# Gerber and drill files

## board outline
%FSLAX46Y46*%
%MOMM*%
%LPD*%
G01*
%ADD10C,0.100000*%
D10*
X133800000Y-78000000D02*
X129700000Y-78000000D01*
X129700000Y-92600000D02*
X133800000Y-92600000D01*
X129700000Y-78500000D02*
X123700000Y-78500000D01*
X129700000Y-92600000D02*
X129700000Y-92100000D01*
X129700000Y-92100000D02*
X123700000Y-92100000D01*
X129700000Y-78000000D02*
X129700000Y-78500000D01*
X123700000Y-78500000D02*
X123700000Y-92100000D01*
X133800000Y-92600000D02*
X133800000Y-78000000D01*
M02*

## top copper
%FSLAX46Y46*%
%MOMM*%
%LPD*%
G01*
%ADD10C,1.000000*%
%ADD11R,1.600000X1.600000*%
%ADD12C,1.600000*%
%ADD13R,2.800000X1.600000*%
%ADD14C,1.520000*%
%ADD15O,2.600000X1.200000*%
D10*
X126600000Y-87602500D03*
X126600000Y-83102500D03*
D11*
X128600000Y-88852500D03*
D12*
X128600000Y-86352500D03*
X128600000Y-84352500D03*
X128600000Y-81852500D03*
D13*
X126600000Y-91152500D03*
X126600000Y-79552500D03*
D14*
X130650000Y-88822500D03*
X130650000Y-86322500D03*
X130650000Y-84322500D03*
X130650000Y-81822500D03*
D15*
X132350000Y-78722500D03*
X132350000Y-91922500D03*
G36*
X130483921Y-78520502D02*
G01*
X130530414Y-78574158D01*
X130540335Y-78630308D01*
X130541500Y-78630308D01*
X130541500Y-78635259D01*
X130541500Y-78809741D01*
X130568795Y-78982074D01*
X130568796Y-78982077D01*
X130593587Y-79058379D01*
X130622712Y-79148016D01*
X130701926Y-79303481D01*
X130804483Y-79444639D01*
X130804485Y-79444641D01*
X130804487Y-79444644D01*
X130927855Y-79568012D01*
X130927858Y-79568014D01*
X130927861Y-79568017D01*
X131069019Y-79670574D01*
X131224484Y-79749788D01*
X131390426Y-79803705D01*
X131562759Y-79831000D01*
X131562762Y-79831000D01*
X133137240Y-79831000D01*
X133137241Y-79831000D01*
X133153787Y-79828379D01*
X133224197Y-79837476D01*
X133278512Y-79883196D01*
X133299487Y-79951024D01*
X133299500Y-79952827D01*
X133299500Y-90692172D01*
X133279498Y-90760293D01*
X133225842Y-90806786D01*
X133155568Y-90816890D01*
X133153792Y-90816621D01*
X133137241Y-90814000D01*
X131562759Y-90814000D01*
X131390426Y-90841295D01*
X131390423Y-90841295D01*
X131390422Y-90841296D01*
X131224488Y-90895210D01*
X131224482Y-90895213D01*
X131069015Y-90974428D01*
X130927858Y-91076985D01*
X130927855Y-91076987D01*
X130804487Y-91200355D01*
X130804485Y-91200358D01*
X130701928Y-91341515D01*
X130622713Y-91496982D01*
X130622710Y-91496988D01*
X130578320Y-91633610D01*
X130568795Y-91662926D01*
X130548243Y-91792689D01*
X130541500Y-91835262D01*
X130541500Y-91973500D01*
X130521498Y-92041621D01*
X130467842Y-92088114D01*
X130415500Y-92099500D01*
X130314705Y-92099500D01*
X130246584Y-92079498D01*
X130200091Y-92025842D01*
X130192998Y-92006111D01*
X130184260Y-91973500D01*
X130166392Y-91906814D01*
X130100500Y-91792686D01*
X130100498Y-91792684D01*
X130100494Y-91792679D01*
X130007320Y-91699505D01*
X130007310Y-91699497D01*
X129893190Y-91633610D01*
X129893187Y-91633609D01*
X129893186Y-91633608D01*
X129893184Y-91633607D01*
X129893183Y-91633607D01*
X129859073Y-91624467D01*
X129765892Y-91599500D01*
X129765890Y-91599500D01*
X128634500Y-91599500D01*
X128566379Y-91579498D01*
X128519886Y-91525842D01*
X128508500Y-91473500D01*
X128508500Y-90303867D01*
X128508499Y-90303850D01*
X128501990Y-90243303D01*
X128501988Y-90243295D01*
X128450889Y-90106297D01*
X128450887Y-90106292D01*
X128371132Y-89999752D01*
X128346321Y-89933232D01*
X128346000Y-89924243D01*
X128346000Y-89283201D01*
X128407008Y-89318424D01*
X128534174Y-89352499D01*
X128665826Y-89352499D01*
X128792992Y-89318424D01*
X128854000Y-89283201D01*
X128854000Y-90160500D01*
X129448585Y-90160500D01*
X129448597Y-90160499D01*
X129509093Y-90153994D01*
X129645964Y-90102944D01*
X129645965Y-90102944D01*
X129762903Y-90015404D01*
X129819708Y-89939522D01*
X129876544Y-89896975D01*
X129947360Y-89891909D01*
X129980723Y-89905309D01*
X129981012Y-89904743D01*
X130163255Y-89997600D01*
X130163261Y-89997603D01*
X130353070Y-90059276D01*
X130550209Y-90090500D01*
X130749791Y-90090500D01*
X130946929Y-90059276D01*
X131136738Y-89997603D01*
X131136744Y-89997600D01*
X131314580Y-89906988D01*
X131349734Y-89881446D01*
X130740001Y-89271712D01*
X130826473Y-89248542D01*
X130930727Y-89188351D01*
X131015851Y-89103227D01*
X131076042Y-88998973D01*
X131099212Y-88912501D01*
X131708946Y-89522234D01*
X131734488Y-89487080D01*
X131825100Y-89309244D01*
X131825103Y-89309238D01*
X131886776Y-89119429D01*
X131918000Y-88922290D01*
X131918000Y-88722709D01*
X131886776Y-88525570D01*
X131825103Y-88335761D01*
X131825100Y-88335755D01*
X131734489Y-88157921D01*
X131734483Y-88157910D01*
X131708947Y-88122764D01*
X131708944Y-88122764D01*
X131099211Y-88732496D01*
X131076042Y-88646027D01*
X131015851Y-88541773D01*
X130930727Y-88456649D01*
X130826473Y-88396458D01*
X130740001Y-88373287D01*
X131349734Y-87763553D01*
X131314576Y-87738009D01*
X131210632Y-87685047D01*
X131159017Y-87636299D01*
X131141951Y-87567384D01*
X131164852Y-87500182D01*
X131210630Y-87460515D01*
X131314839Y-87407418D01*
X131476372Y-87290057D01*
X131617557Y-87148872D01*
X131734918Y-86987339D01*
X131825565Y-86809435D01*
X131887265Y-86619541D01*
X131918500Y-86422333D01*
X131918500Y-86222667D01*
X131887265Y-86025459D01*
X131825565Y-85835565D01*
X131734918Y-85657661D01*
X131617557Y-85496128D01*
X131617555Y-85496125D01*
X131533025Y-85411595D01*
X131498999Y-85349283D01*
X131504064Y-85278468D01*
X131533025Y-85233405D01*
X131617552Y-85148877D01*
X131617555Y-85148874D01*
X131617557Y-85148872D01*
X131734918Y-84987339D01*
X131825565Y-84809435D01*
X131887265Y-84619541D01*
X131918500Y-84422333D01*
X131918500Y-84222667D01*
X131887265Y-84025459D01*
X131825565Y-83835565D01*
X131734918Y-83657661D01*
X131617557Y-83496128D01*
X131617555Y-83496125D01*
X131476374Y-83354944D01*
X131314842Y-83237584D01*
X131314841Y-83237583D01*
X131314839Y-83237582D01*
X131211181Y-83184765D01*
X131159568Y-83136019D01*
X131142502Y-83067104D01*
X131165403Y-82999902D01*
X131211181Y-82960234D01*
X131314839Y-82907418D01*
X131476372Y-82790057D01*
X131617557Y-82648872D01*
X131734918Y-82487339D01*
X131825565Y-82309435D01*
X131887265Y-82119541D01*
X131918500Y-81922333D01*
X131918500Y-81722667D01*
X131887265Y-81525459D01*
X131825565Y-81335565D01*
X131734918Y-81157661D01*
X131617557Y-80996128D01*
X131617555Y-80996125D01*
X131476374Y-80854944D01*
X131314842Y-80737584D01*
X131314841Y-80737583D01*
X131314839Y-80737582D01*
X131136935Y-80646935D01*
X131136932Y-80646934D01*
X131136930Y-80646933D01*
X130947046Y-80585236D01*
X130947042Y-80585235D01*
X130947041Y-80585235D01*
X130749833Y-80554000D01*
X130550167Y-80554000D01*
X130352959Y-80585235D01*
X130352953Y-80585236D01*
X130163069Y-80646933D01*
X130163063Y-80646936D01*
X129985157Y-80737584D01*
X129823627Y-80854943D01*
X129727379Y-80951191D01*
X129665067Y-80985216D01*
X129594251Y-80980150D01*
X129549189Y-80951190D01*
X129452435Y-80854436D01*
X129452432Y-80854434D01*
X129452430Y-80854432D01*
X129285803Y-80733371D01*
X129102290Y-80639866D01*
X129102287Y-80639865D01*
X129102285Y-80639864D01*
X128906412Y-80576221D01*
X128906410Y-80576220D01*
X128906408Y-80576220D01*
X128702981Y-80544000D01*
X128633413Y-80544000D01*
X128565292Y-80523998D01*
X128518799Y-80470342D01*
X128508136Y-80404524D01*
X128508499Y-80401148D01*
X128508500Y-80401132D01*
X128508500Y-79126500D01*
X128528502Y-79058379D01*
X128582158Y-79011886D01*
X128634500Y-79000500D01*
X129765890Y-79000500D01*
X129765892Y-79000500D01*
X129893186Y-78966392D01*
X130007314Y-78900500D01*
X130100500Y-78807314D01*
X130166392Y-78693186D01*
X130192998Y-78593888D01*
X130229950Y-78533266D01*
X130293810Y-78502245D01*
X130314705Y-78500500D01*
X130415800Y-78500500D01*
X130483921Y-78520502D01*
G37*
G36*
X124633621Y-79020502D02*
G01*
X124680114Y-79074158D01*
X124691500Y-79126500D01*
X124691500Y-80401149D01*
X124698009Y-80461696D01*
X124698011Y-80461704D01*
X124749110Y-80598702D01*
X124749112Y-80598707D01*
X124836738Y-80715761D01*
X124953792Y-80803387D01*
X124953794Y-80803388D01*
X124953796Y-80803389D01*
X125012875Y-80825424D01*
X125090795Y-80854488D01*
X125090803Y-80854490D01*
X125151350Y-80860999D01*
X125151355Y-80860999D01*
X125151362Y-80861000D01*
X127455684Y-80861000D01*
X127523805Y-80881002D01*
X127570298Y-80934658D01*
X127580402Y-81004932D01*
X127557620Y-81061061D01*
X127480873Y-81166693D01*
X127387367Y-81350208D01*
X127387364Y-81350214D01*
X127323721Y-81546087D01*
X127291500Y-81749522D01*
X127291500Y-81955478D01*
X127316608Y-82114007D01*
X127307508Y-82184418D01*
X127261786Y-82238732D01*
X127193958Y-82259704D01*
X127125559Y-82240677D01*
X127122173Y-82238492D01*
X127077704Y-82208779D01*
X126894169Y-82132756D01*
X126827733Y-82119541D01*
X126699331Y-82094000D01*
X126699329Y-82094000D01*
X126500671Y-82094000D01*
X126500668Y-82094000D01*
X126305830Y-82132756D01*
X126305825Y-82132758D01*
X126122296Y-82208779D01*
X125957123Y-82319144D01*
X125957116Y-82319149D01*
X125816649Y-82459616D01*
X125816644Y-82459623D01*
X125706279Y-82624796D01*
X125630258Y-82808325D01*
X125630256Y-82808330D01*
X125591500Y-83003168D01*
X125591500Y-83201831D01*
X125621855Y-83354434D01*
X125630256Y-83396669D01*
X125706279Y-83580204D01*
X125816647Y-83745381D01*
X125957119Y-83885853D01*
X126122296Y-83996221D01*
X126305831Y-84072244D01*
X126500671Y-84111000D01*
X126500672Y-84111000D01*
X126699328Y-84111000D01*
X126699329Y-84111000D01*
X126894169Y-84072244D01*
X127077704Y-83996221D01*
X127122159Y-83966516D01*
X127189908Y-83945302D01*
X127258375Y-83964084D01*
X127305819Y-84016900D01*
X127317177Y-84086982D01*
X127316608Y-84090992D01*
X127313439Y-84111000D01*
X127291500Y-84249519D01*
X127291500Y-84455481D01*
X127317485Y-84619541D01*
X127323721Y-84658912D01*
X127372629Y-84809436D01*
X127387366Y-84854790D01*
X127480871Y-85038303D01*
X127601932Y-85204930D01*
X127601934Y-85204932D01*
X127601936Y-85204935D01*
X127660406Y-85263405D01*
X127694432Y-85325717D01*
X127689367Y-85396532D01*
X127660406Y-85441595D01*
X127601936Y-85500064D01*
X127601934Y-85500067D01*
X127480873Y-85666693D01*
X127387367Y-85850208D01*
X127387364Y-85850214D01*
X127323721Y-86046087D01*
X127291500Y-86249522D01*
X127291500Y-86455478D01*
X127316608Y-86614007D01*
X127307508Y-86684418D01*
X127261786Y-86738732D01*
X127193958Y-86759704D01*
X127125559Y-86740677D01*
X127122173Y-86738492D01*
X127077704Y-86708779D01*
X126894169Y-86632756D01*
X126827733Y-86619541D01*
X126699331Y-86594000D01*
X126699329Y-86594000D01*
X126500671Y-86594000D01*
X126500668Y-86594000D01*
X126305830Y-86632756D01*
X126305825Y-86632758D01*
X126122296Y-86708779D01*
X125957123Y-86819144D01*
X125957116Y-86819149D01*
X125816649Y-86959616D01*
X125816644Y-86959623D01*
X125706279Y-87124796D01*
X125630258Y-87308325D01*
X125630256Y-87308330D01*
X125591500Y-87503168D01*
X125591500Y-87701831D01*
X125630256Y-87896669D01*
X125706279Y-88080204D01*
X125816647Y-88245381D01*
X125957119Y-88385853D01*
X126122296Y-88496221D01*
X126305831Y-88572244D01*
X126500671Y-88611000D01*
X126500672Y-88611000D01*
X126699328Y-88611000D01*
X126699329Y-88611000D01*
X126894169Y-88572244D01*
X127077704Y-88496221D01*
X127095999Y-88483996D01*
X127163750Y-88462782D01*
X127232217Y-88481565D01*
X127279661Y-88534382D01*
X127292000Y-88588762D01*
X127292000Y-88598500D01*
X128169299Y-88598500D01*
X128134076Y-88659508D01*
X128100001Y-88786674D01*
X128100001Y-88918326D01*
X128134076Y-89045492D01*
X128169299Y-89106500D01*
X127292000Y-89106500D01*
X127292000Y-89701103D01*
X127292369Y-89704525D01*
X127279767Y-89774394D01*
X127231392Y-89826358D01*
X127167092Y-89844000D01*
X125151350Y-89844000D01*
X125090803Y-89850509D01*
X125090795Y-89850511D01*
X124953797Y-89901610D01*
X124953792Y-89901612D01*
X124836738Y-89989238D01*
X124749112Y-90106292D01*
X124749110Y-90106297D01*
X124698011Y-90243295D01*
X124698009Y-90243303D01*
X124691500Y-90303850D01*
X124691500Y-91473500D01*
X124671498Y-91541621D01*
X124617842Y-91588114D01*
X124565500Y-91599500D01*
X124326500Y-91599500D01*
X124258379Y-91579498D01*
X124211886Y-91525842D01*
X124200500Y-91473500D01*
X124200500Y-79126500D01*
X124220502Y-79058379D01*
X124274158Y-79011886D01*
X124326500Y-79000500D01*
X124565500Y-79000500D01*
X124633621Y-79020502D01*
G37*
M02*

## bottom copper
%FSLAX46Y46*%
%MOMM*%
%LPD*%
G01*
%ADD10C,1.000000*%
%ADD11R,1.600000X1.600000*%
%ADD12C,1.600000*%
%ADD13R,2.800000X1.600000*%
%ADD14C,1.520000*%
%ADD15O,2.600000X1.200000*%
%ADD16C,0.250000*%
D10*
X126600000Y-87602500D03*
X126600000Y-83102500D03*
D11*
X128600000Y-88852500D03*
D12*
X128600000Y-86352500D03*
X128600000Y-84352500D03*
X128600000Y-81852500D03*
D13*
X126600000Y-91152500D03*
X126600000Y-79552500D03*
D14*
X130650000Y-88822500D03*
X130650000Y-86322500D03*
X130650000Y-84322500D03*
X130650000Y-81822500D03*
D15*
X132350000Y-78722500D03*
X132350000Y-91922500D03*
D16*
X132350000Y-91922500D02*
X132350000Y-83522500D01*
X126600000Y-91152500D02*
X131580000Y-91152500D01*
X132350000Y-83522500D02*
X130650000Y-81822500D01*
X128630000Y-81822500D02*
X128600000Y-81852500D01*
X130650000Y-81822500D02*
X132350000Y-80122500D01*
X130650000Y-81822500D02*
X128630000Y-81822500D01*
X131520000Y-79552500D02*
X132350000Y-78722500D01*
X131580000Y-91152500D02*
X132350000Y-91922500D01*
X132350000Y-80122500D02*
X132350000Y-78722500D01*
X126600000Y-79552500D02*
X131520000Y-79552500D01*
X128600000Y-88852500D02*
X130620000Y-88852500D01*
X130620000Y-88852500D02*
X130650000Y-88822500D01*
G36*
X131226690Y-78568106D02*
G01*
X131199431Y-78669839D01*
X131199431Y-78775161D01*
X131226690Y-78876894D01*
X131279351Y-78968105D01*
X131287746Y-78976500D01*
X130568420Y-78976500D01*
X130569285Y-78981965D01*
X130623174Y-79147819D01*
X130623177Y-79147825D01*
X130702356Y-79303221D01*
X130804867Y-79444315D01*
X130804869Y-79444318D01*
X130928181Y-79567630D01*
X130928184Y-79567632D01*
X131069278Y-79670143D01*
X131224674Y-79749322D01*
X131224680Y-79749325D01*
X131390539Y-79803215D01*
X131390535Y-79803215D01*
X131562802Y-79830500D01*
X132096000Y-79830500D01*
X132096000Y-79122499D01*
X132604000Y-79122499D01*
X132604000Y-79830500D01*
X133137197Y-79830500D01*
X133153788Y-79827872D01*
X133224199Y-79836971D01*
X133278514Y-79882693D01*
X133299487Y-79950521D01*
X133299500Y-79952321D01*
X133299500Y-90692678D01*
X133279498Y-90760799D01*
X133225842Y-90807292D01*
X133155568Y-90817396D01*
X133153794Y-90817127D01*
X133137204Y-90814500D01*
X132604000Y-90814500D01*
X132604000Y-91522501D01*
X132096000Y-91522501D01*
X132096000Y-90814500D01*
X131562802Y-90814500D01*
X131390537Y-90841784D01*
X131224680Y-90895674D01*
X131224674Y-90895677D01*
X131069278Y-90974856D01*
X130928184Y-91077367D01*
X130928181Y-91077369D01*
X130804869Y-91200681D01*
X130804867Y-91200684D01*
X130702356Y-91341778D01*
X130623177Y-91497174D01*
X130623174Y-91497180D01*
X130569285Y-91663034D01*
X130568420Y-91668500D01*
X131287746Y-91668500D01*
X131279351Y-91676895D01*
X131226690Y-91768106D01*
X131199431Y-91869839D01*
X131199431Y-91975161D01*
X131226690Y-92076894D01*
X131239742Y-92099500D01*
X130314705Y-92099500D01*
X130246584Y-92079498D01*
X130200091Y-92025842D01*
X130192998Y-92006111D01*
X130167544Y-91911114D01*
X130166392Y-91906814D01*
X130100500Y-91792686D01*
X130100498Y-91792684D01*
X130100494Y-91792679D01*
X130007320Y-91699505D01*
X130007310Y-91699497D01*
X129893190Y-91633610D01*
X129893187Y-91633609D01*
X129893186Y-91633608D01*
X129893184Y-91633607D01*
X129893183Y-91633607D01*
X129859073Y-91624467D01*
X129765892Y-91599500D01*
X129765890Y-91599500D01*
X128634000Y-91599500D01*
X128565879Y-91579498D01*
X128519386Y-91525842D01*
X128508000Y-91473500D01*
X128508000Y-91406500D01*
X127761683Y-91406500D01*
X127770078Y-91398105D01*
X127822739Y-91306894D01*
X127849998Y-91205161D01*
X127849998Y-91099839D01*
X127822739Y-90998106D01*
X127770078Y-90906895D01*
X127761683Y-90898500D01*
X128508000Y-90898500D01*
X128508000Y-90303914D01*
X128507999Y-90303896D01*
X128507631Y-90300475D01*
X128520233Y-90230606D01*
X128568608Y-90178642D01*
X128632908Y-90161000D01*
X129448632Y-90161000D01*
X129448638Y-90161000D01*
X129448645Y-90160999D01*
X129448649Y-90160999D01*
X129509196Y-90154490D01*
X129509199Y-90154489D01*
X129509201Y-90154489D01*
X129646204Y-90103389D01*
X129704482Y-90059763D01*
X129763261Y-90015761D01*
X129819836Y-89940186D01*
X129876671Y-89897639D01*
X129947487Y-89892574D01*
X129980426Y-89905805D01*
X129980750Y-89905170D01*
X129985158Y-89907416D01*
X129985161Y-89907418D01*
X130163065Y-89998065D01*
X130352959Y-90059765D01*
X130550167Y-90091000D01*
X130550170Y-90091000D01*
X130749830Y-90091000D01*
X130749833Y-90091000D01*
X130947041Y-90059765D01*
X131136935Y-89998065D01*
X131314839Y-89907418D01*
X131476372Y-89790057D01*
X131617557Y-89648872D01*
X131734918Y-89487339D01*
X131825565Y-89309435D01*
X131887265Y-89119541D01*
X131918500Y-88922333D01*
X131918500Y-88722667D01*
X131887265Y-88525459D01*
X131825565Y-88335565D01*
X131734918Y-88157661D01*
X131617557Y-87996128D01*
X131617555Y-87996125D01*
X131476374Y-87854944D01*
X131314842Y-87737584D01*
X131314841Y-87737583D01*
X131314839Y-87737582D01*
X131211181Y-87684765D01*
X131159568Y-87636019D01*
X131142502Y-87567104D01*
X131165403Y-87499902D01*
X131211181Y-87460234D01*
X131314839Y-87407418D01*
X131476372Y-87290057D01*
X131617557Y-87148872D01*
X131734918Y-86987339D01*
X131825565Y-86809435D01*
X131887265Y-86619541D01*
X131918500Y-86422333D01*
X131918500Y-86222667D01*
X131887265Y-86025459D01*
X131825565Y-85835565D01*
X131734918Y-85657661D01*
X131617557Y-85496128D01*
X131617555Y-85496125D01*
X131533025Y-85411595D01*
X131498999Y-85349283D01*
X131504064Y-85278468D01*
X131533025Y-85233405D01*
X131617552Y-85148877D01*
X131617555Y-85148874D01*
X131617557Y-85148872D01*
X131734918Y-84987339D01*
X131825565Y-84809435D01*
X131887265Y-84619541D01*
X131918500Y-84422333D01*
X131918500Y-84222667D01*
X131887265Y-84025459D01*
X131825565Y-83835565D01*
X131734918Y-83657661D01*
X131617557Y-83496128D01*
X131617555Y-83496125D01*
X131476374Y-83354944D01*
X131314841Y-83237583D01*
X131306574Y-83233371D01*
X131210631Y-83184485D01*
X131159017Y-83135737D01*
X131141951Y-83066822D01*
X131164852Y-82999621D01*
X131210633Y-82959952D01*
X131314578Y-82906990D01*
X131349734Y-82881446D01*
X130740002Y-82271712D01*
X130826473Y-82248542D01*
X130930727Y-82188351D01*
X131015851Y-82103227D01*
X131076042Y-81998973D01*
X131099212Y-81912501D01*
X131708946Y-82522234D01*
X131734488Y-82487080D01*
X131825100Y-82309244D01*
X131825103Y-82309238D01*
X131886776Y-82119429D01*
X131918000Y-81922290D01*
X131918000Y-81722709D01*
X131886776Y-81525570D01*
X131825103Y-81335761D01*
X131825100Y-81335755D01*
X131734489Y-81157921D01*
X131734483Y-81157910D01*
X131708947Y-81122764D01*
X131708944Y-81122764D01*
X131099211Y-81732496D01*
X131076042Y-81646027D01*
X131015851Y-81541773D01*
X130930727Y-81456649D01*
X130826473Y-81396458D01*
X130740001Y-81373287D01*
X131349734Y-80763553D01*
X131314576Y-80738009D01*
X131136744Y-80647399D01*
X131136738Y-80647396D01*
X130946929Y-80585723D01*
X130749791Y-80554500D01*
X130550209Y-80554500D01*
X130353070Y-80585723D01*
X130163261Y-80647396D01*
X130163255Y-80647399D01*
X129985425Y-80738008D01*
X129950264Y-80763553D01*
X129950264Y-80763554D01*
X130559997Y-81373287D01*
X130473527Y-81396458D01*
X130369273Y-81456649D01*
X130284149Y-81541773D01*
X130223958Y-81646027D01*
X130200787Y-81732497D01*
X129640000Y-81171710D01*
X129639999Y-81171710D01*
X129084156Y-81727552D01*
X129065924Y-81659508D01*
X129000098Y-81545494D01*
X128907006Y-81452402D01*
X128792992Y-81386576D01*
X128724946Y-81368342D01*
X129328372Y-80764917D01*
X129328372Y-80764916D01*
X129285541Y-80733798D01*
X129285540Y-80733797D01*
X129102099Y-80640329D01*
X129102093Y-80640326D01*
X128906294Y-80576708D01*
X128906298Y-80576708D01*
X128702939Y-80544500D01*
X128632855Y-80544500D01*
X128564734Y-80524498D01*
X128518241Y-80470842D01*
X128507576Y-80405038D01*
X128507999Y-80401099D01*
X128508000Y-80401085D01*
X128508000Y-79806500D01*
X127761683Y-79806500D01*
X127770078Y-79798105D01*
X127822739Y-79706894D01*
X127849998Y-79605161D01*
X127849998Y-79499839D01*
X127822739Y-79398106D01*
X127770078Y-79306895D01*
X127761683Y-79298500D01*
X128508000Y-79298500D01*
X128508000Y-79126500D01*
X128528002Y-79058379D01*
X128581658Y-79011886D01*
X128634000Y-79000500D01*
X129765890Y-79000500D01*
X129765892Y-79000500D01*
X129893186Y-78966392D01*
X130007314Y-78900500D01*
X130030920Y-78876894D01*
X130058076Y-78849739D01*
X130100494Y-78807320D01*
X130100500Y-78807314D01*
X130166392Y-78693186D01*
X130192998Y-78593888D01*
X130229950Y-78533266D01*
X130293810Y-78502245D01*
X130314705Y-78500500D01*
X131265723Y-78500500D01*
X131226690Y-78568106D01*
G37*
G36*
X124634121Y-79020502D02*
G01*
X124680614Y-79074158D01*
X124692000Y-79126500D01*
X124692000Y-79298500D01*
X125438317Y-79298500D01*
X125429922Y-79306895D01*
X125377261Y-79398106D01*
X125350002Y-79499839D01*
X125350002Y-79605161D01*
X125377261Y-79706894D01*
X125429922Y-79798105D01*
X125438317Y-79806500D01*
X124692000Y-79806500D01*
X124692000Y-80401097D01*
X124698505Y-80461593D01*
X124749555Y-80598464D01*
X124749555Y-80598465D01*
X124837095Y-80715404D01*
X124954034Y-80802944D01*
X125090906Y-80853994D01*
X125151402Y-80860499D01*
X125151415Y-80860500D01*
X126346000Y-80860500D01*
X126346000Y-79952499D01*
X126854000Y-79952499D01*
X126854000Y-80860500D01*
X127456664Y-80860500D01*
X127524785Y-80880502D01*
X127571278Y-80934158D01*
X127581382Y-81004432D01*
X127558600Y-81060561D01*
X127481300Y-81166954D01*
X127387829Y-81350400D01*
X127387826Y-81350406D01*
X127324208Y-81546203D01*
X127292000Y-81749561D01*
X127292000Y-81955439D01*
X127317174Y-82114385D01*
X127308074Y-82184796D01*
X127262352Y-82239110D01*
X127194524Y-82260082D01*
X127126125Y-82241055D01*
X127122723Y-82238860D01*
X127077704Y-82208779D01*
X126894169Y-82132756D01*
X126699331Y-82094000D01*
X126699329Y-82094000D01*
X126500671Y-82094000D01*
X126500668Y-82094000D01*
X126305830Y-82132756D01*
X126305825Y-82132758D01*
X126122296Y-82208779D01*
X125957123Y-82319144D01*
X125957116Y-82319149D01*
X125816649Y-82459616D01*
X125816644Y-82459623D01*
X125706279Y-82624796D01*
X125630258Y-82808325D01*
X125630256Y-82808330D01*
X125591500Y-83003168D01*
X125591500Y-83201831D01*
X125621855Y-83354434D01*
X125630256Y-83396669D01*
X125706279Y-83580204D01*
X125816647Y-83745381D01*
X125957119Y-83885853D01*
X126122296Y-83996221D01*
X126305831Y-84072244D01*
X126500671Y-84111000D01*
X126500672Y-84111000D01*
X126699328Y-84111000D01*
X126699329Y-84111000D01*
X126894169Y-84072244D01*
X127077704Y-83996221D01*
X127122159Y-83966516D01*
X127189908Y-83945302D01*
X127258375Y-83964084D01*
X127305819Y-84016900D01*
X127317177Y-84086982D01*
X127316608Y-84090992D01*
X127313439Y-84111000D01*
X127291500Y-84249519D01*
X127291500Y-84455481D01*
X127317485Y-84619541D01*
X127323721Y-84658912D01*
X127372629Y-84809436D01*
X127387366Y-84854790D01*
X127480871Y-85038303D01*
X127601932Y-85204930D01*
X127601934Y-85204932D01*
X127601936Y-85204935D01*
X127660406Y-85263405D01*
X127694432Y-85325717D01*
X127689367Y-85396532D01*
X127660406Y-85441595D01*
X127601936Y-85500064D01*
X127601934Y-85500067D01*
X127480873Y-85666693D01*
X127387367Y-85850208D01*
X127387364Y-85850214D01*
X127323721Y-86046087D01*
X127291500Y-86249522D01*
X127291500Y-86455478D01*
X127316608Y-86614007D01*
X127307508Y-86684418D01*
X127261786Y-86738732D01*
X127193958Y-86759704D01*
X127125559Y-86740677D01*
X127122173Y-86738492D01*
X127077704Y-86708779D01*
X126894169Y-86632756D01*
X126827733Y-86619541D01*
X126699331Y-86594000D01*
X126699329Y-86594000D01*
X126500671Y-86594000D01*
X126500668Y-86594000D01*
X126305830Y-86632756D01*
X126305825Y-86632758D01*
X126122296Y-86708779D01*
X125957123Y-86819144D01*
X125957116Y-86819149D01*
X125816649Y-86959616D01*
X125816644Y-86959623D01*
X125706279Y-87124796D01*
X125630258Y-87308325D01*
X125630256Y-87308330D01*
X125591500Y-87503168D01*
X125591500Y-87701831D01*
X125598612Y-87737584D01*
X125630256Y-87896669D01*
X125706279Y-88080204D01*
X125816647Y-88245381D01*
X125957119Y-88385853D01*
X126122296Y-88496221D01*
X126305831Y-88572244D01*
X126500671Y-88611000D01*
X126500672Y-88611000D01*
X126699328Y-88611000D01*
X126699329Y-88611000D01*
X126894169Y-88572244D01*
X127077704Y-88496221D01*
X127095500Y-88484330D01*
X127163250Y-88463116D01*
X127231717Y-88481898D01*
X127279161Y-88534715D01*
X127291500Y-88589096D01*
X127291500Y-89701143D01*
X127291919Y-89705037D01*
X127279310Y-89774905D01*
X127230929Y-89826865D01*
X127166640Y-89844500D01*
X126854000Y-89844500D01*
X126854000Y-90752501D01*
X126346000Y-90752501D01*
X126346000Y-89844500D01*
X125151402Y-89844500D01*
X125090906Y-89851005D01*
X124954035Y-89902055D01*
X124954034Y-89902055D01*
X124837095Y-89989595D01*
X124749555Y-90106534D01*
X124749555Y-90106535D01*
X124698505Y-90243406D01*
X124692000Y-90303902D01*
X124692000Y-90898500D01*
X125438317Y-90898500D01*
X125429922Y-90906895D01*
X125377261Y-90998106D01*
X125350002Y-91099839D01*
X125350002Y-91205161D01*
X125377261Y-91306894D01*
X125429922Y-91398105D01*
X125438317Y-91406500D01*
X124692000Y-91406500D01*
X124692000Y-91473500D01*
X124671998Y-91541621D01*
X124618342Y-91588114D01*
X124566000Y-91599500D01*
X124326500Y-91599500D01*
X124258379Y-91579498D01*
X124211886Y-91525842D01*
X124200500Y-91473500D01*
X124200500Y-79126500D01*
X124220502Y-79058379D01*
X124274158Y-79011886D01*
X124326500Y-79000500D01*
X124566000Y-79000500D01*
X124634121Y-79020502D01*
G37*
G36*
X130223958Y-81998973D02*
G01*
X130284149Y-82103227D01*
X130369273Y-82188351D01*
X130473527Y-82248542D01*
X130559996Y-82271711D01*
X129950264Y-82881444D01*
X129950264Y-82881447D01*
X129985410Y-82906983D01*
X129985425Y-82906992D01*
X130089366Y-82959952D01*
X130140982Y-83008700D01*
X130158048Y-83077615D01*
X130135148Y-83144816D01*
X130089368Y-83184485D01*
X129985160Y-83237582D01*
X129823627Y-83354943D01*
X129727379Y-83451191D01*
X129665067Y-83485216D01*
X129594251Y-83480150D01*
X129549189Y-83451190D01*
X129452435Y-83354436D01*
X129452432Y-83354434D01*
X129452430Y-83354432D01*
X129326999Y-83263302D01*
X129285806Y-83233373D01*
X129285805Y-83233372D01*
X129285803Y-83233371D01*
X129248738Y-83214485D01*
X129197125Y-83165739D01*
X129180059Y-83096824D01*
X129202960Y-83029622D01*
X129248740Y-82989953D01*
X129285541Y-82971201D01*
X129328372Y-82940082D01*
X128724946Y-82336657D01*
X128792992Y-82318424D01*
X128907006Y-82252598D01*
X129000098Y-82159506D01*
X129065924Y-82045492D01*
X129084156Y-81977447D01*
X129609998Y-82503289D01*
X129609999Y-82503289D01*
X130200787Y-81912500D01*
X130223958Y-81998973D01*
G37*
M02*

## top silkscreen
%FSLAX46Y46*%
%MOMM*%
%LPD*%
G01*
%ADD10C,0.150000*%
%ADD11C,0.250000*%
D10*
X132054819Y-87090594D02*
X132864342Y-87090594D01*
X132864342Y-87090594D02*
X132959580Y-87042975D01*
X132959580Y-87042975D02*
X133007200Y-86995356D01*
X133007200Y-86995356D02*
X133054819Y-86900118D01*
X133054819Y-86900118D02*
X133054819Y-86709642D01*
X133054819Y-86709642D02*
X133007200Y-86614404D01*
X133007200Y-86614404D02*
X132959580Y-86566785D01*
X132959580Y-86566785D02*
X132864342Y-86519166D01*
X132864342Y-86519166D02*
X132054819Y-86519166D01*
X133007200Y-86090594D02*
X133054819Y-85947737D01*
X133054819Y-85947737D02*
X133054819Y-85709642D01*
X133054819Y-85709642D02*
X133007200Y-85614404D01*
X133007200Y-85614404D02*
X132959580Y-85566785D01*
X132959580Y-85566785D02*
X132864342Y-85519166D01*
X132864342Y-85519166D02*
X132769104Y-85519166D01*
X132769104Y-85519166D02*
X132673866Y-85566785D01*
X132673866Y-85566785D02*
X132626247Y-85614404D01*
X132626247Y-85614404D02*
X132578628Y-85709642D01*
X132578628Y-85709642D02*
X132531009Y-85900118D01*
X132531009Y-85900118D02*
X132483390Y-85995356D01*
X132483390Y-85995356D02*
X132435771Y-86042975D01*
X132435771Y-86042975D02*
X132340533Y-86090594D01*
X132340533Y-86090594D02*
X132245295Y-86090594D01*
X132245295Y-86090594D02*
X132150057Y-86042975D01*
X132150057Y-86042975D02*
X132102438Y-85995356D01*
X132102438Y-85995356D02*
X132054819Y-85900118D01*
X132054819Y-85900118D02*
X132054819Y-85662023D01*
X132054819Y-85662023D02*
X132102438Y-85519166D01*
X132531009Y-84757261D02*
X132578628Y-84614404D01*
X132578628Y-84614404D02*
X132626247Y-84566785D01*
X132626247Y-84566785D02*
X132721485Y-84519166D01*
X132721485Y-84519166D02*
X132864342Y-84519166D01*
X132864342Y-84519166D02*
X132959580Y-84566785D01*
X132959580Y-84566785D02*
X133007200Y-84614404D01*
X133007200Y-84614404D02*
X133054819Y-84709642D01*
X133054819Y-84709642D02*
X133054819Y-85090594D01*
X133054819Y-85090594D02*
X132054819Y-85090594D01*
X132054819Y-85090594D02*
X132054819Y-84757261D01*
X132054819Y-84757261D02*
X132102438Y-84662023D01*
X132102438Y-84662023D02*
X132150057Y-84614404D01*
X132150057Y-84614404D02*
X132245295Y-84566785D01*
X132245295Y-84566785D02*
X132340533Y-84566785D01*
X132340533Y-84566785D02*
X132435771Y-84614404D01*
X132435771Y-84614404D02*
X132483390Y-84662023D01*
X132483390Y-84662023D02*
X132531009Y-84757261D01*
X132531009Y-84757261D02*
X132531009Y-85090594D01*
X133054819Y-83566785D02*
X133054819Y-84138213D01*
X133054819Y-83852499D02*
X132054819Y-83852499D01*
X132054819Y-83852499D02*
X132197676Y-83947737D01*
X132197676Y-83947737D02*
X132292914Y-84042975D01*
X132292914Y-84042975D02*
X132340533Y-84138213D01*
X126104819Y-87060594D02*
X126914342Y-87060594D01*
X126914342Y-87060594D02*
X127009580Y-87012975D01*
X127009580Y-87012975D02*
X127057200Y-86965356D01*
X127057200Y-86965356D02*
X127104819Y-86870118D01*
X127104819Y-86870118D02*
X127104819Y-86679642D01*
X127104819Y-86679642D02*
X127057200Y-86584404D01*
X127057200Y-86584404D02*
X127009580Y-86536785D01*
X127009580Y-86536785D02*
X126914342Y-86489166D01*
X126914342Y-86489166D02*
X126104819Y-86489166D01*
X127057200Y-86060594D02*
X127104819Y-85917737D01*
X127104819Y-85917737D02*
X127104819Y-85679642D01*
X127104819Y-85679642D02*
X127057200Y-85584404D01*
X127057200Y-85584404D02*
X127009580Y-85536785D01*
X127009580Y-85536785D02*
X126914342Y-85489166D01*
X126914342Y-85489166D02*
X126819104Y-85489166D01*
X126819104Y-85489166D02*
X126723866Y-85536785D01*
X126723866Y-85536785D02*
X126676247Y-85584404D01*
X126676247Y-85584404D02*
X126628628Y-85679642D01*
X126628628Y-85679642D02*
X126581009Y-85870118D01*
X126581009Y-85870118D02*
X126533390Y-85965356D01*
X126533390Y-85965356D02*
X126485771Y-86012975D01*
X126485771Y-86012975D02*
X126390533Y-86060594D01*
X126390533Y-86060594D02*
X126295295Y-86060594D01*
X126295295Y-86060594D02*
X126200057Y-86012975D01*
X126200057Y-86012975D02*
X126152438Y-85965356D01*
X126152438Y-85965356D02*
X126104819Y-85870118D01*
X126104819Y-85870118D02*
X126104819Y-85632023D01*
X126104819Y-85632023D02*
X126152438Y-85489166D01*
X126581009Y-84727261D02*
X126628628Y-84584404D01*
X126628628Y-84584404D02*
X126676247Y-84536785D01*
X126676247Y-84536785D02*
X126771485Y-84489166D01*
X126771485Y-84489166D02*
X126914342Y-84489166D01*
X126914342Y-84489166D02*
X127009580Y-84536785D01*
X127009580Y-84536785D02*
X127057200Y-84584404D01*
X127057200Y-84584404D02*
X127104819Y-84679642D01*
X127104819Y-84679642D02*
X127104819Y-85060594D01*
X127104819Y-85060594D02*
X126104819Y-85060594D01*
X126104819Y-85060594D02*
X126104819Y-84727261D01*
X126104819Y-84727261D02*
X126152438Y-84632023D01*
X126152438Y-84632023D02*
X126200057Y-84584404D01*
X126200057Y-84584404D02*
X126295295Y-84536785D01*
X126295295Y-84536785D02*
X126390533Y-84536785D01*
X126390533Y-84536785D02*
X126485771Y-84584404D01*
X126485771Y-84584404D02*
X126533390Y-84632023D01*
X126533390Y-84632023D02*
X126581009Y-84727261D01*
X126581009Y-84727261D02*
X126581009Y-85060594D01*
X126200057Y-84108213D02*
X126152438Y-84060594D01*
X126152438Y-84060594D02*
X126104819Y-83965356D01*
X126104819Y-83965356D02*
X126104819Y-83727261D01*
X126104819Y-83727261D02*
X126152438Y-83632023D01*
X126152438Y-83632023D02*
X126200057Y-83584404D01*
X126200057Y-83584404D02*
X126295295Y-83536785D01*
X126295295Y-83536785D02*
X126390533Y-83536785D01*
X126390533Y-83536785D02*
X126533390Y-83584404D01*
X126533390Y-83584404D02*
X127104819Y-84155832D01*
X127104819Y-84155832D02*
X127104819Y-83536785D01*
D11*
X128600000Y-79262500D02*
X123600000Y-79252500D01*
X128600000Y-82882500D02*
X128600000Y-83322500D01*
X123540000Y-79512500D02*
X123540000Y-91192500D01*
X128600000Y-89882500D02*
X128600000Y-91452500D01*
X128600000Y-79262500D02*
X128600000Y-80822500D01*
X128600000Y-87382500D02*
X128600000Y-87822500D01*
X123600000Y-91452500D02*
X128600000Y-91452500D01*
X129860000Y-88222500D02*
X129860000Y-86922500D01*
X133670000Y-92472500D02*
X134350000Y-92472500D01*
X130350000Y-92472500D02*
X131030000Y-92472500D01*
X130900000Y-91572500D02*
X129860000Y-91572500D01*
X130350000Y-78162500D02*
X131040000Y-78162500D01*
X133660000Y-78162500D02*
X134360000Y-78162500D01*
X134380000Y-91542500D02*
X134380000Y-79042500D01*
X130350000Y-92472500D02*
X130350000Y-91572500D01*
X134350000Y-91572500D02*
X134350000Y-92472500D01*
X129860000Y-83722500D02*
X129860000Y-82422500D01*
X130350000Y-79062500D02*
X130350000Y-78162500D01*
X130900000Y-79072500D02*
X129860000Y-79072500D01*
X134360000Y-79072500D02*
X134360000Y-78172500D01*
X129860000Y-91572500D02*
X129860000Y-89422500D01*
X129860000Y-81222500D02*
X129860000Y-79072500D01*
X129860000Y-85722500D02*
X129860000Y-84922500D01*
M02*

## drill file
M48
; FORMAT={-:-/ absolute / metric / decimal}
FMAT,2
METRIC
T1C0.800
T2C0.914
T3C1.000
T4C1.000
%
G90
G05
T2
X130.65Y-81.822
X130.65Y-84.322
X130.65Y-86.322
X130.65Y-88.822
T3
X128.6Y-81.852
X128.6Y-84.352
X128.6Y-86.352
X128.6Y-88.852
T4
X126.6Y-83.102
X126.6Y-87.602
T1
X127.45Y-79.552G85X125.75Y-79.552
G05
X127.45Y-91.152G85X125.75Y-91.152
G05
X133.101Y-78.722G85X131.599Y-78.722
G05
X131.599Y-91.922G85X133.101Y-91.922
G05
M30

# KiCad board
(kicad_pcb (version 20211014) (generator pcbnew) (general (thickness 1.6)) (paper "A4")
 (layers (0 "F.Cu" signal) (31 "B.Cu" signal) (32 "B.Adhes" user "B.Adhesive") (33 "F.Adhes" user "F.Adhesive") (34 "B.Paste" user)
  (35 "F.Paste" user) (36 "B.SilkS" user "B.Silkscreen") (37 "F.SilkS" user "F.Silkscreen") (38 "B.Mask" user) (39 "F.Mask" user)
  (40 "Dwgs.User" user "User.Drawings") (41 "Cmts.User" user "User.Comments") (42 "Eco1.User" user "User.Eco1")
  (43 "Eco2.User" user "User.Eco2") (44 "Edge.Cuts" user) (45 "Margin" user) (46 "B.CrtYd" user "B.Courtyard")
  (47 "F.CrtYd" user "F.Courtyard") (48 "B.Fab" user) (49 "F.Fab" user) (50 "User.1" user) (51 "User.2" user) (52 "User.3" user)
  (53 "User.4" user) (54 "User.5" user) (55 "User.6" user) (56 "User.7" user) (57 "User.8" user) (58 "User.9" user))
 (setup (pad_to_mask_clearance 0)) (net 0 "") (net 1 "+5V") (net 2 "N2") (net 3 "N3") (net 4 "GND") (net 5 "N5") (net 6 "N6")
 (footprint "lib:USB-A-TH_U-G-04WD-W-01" (layer "F.Cu") (at 127.6 85.3525 -90)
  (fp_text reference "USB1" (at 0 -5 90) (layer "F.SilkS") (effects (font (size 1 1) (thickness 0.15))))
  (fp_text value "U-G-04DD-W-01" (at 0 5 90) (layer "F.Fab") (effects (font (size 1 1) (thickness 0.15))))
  (fp_line (start -6.09 -1) (end -6.1 4) (layer "F.SilkS") (width 0.25))
  (fp_line (start -2.47 -1) (end -2.03 -1) (layer "F.SilkS") (width 0.25))
  (fp_line (start -5.84 4.06) (end 5.84 4.06) (layer "F.SilkS") (width 0.25))
  (fp_line (start 4.53 -1) (end 6.1 -1) (layer "F.SilkS") (width 0.25))
  (fp_line (start -6.09 -1) (end -4.53 -1) (layer "F.SilkS") (width 0.25))
  (fp_line (start 2.03 -1) (end 2.47 -1) (layer "F.SilkS") (width 0.25))
  (fp_line (start 6.1 4) (end 6.1 -1) (layer "F.SilkS") (width 0.25))
  (pad "" thru_hole circle (at 2.25 1 270) (size 1 1) (drill 1) (layers *.Cu *.Mask))
  (pad "" thru_hole circle (at -2.25 1 270) (size 1 1) (drill 1) (layers *.Cu *.Mask))
  (pad "1" thru_hole rect (at 3.5 -1 270) (size 1.6 1.6) (drill 0.999998) (layers *.Cu *.Paste *.Mask) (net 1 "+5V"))
  (pad "2" thru_hole circle (at 1 -1 270) (size 1.6 1.6) (drill 0.999998) (layers *.Cu *.Paste *.Mask) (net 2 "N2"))
  (pad "3" thru_hole circle (at -1 -1 270) (size 1.6 1.6) (drill 0.999998) (layers *.Cu *.Paste *.Mask) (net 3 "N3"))
  (pad "4" thru_hole circle (at -3.5 -1 270) (size 1.6 1.6) (drill 0.999998) (layers *.Cu *.Paste *.Mask) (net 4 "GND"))
  (pad "5" thru_hole rect (at 5.8 1 270) (size 1.6 2.8) (drill oval 0.799998 2.499995) (layers *.Cu *.Paste *.Mask) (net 4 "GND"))
  (pad "6" thru_hole rect (at -5.8 1 270) (size 1.6 2.8) (drill oval 0.799998 2.499995) (layers *.Cu *.Paste *.Mask) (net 4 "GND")))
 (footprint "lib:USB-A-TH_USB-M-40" (layer "F.Cu") (at 131.5 85.3225 90)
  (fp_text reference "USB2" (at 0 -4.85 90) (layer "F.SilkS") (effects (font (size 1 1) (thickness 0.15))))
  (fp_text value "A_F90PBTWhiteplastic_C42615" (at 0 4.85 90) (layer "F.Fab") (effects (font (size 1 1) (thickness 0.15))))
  (fp_line (start -2.9 -1.64) (end -1.6 -1.64) (layer "F.SilkS") (width 0.25))
  (fp_line (start -7.15 2.17) (end -7.15 2.85) (layer "F.SilkS") (width 0.25))
  (fp_line (start -7.15 -1.15) (end -7.15 -0.47) (layer "F.SilkS") (width 0.25))
  (fp_line (start -6.25 -0.6) (end -6.25 -1.64) (layer "F.SilkS") (width 0.25))
  (fp_line (start 7.16 -1.15) (end 7.16 -0.46) (layer "F.SilkS") (width 0.25))
  (fp_line (start 7.16 2.16) (end 7.16 2.86) (layer "F.SilkS") (width 0.25))
  (fp_line (start -6.22 2.88) (end 6.28 2.88) (layer "F.SilkS") (width 0.25))
  (fp_line (start -7.15 -1.15) (end -6.25 -1.15) (layer "F.SilkS") (width 0.25))
  (fp_line (start -6.25 2.85) (end -7.15 2.85) (layer "F.SilkS") (width 0.25))
  (fp_line (start 1.6 -1.64) (end 2.9 -1.64) (layer "F.SilkS") (width 0.25))
  (fp_line (start 6.26 -1.15) (end 7.16 -1.15) (layer "F.SilkS") (width 0.25))
  (fp_line (start 6.25 -0.6) (end 6.25 -1.64) (layer "F.SilkS") (width 0.25))
  (fp_line (start 6.25 2.86) (end 7.15 2.86) (layer "F.SilkS") (width 0.25))
  (fp_line (start -6.25 -1.64) (end -4.1 -1.64) (layer "F.SilkS") (width 0.25))
  (fp_line (start 4.1 -1.64) (end 6.25 -1.64) (layer "F.SilkS") (width 0.25))
  (fp_line (start -0.4 -1.64) (end 0.4 -1.64) (layer "F.SilkS") (width 0.25))
  (pad "1" thru_hole circle (at -3.5 -0.85 90) (size 1.52 1.52) (drill 0.9144) (layers *.Cu *.Paste *.Mask) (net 1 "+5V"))
  (pad "2" thru_hole circle (at -1 -0.85 90) (size 1.52 1.52) (drill 0.9144) (layers *.Cu *.Paste *.Mask) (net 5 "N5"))
  (pad "3" thru_hole circle (at 1 -0.85 90) (size 1.52 1.52) (drill 0.9144) (layers *.Cu *.Paste *.Mask) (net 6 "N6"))
  (pad "4" thru_hole circle (at 3.5 -0.85 90) (size 1.52 1.52) (drill 0.9144) (layers *.Cu *.Paste *.Mask) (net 4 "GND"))
  (pad "5" thru_hole oval (at 6.6 0.85 180) (size 2.6 1.2) (drill oval 2.301138 0.799998) (layers *.Cu *.Paste *.Mask) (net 4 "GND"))
  (pad "6" thru_hole oval (at -6.6 0.85) (size 2.6 1.2) (drill oval 2.301138 0.799998) (layers *.Cu *.Paste *.Mask) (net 4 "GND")))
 (gr_line (start 133.8 78) (end 129.7 78) (layer "Edge.Cuts") (width 0.1))
 (gr_line (start 129.7 92.6) (end 133.8 92.6) (layer "Edge.Cuts") (width 0.1))
 (gr_line (start 129.7 78.5) (end 123.7 78.5) (layer "Edge.Cuts") (width 0.1))
 (gr_line (start 129.7 92.6) (end 129.7 92.1) (layer "Edge.Cuts") (width 0.1))
 (gr_line (start 129.7 92.1) (end 123.7 92.1) (layer "Edge.Cuts") (width 0.1))
 (gr_line (start 129.7 78) (end 129.7 78.5) (layer "Edge.Cuts") (width 0.1))
 (gr_line (start 123.7 78.5) (end 123.7 92.1) (layer "Edge.Cuts") (width 0.1))
 (gr_line (start 133.8 92.6) (end 133.8 78) (layer "Edge.Cuts") (width 0.1))
 (segment (start 132.35 91.9225) (end 132.35 83.5225) (width 0.25) (layer "B.Cu") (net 4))
 (segment (start 126.6 91.1525) (end 131.58 91.1525) (width 0.25) (layer "B.Cu") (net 4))
 (segment (start 132.35 83.5225) (end 130.65 81.8225) (width 0.25) (layer "B.Cu") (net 4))
 (segment (start 128.63 81.8225) (end 128.6 81.8525) (width 0.25) (layer "B.Cu") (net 4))
 (segment (start 130.65 81.8225) (end 132.35 80.1225) (width 0.25) (layer "B.Cu") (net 4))
 (segment (start 130.65 81.8225) (end 128.63 81.8225) (width 0.25) (layer "B.Cu") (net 4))
 (segment (start 131.52 79.5525) (end 132.35 78.7225) (width 0.25) (layer "B.Cu") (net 4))
 (segment (start 131.58 91.1525) (end 132.35 91.9225) (width 0.25) (layer "B.Cu") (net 4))
 (segment (start 132.35 80.1225) (end 132.35 78.7225) (width 0.25) (layer "B.Cu") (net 4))
 (segment (start 126.6 79.5525) (end 131.52 79.5525) (width 0.25) (layer "B.Cu") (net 4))
 (segment (start 128.6 88.8525) (end 130.62 88.8525) (width 0.25) (layer "B.Cu") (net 1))
 (segment (start 130.62 88.8525) (end 130.65 88.8225) (width 0.25) (layer "B.Cu") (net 1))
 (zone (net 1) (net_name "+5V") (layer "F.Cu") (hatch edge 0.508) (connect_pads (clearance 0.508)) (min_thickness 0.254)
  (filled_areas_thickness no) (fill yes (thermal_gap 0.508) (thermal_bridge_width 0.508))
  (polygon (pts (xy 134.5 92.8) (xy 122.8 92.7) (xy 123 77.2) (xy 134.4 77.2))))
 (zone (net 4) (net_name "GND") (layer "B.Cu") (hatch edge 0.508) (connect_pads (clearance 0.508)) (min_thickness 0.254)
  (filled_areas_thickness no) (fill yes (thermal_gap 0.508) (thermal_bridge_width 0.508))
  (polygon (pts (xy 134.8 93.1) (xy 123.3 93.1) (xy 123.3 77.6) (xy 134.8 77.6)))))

